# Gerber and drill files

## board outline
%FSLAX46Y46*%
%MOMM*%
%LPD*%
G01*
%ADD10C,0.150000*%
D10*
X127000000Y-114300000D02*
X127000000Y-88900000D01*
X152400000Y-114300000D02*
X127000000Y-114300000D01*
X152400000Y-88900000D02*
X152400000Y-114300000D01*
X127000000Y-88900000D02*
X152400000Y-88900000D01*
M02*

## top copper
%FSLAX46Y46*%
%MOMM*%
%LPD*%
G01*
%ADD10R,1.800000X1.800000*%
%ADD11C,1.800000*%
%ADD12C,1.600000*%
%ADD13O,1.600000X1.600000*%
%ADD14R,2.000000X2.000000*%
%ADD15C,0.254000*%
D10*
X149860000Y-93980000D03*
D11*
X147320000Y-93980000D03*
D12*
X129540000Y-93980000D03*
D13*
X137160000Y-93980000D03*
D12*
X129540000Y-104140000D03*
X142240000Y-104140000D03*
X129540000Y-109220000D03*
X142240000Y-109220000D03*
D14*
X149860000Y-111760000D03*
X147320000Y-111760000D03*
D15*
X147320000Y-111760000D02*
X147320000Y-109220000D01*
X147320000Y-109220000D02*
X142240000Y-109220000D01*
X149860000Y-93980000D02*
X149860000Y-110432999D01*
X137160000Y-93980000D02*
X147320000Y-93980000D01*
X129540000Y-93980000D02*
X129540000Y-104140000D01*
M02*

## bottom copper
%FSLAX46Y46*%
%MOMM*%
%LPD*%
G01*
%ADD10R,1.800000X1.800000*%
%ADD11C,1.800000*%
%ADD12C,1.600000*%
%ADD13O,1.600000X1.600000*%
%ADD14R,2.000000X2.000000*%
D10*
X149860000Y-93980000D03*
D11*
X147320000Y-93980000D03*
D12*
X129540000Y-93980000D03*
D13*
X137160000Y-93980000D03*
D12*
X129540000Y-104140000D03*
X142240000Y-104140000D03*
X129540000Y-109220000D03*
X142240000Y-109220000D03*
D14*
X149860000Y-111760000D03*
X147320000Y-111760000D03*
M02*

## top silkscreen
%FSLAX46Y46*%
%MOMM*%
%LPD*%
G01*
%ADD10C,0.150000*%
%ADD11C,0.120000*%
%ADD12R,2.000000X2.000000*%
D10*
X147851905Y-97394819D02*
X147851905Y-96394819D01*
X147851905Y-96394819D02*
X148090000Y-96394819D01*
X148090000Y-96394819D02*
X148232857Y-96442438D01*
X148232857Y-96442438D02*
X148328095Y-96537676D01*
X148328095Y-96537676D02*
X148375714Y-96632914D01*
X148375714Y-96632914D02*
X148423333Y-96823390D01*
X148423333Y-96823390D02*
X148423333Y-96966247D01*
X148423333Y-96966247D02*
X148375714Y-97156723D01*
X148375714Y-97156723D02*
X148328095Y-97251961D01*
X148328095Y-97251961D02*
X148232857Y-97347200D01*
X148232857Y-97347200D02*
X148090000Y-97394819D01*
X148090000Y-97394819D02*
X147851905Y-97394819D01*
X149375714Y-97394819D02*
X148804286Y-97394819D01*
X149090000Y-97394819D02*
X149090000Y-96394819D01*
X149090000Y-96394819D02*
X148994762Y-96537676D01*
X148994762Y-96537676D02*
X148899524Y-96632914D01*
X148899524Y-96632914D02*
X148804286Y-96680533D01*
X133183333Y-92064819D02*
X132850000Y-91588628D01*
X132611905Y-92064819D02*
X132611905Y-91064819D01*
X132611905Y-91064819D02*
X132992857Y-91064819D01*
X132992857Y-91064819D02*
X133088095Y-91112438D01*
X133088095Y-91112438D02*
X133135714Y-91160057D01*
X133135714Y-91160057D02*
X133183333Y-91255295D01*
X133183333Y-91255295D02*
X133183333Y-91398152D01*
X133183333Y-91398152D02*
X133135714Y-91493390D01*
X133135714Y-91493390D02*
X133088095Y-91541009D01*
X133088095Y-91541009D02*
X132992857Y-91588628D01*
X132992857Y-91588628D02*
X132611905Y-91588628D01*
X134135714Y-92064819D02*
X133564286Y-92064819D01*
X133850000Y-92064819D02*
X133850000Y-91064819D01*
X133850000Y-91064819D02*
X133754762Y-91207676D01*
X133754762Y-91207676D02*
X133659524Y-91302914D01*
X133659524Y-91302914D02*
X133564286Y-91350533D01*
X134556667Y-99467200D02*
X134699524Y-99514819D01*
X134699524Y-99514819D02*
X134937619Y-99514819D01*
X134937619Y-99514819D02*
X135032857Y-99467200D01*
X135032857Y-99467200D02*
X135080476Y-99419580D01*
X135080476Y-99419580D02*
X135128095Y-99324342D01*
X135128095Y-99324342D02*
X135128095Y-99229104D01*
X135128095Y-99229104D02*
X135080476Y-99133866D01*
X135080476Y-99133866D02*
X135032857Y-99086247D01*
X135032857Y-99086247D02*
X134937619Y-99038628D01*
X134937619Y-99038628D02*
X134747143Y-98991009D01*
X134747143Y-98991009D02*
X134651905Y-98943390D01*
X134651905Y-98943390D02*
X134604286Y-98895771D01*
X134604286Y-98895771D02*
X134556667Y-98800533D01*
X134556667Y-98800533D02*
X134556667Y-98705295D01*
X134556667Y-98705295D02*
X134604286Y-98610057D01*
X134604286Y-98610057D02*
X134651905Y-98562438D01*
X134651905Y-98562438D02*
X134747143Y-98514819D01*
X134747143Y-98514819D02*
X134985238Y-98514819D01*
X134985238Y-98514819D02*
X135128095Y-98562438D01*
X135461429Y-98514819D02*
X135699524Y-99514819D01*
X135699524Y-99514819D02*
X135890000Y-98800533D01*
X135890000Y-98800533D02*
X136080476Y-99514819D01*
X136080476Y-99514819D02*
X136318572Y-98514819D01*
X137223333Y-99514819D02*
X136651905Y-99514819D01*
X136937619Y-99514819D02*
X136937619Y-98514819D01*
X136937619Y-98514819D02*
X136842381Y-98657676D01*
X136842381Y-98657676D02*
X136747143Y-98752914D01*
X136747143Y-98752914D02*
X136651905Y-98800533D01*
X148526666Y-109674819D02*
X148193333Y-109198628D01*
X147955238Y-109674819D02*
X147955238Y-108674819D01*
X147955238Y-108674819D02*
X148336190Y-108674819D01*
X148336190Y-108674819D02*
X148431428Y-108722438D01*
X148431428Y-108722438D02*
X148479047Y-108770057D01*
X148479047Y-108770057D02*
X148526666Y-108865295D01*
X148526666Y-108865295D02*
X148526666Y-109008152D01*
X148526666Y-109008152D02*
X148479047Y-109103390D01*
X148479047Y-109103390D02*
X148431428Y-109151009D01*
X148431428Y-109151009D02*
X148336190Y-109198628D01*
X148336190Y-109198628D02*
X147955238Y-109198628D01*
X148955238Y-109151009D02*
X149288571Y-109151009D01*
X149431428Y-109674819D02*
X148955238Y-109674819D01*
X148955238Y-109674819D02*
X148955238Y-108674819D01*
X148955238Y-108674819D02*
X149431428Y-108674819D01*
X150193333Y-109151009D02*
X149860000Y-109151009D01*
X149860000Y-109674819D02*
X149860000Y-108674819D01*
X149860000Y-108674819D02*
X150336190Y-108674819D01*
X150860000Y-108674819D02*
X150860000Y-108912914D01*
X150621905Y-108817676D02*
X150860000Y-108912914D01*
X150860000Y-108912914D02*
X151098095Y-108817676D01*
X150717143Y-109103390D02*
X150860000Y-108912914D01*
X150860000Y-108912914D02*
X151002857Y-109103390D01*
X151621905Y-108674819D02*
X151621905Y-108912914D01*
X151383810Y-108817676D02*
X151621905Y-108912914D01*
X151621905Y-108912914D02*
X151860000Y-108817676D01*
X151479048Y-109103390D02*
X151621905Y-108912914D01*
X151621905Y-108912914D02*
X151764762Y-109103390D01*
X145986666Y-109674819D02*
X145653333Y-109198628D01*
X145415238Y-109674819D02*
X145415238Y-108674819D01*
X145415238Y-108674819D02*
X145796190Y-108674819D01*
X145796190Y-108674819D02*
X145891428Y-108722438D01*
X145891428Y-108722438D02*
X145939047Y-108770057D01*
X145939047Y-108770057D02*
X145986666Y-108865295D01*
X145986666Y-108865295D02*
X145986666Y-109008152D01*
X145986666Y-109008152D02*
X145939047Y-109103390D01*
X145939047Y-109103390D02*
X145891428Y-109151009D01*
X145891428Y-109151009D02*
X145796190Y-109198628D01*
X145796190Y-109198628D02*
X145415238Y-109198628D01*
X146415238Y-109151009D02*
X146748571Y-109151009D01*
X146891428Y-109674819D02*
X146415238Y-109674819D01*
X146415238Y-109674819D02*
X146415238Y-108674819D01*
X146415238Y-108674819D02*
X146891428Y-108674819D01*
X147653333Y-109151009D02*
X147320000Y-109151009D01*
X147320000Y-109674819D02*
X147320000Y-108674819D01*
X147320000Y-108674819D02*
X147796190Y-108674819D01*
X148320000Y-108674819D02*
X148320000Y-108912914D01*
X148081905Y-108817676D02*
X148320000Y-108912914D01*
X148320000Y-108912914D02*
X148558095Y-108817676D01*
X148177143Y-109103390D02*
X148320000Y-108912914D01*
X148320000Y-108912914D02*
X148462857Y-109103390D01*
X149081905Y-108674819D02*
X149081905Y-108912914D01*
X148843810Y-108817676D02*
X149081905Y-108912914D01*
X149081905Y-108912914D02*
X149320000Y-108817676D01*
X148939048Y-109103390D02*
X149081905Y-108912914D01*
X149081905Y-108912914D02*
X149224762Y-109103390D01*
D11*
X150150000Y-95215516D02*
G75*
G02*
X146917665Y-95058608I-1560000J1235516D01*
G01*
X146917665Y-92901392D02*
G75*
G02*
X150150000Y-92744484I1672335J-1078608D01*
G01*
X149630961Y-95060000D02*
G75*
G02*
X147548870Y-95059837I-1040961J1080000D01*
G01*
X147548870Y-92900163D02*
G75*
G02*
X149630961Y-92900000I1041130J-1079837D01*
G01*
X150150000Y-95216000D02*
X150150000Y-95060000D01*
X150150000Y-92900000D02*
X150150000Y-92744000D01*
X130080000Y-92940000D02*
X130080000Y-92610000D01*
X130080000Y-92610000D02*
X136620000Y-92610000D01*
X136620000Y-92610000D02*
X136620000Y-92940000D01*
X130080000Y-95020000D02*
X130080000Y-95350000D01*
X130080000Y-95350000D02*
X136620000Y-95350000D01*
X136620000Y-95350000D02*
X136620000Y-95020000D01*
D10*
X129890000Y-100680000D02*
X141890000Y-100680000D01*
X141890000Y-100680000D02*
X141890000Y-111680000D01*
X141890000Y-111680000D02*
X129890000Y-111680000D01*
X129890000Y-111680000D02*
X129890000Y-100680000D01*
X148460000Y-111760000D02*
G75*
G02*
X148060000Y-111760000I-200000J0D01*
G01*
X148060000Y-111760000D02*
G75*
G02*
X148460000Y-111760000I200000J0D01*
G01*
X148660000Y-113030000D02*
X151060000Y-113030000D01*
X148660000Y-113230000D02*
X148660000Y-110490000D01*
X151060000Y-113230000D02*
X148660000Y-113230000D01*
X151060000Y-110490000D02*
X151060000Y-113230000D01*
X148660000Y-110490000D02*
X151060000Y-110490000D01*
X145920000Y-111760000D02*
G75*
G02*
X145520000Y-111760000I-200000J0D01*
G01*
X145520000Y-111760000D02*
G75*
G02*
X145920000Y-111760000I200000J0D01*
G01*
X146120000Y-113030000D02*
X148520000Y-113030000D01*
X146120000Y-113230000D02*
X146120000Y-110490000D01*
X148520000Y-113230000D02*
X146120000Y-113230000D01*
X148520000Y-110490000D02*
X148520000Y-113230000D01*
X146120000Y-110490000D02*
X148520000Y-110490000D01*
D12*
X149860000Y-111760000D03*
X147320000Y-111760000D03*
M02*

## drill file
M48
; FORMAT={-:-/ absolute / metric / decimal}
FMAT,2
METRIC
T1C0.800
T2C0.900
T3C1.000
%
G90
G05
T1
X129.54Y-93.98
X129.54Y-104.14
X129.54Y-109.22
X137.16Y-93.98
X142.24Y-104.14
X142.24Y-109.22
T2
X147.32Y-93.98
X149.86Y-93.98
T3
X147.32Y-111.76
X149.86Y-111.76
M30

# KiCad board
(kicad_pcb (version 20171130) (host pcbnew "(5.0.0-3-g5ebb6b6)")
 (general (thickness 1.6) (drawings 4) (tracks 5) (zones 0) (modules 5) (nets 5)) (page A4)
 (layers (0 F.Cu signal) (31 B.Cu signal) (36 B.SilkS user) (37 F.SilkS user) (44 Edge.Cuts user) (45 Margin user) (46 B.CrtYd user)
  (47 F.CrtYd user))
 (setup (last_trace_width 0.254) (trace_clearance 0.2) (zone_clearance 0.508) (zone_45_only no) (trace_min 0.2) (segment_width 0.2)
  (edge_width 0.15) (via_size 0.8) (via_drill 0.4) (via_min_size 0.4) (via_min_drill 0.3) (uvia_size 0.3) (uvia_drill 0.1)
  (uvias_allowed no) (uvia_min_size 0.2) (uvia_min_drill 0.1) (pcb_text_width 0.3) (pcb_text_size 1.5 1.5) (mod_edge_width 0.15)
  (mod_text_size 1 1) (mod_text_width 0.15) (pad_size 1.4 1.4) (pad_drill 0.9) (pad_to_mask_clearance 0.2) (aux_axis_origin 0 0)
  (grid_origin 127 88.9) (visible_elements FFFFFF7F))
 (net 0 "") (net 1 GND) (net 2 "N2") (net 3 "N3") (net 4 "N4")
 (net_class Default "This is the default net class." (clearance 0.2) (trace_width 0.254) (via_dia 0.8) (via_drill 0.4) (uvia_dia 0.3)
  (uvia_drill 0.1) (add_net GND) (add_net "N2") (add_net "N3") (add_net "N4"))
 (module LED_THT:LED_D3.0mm (layer F.Cu) (at 149.86 93.98 180)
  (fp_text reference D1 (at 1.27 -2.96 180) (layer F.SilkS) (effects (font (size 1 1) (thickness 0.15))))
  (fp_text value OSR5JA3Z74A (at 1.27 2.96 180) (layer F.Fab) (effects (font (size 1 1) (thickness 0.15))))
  (fp_arc (start 1.27 0) (end -0.29 -1.235516) (angle 108.8) (layer F.SilkS) (width 0.12))
  (fp_arc (start 1.27 0) (end -0.29 1.235516) (angle -108.8) (layer F.SilkS) (width 0.12))
  (fp_arc (start 1.27 0) (end 0.229039 -1.08) (angle 87.9) (layer F.SilkS) (width 0.12))
  (fp_arc (start 1.27 0) (end 0.229039 1.08) (angle -87.9) (layer F.SilkS) (width 0.12))
  (fp_line (start -0.29 -1.236) (end -0.29 -1.08) (layer F.SilkS) (width 0.12))
  (fp_line (start -0.29 1.08) (end -0.29 1.236) (layer F.SilkS) (width 0.12))
  (pad 1 thru_hole rect (at 0 0 180) (size 1.8 1.8) (drill 0.9) (layers *.Cu *.Mask) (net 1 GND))
  (pad 2 thru_hole circle (at 2.54 0 180) (size 1.8 1.8) (drill 0.9) (layers *.Cu *.Mask) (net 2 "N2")))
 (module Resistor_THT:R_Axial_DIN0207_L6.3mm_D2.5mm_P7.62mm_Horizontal (layer F.Cu) (at 129.54 93.98)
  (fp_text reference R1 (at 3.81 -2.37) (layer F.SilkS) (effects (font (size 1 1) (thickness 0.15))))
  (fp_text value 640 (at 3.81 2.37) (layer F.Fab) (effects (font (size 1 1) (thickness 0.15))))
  (fp_line (start 0.54 -1.04) (end 0.54 -1.37) (layer F.SilkS) (width 0.12))
  (fp_line (start 0.54 -1.37) (end 7.08 -1.37) (layer F.SilkS) (width 0.12))
  (fp_line (start 7.08 -1.37) (end 7.08 -1.04) (layer F.SilkS) (width 0.12))
  (fp_line (start 0.54 1.04) (end 0.54 1.37) (layer F.SilkS) (width 0.12))
  (fp_line (start 0.54 1.37) (end 7.08 1.37) (layer F.SilkS) (width 0.12))
  (fp_line (start 7.08 1.37) (end 7.08 1.04) (layer F.SilkS) (width 0.12))
  (pad 1 thru_hole circle (at 0 0) (size 1.6 1.6) (drill 0.8) (layers *.Cu *.Mask) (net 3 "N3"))
  (pad 2 thru_hole oval (at 7.62 0) (size 1.6 1.6) (drill 0.8) (layers *.Cu *.Mask) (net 2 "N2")))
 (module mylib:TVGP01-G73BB (layer F.Cu) (at 135.89 106.68)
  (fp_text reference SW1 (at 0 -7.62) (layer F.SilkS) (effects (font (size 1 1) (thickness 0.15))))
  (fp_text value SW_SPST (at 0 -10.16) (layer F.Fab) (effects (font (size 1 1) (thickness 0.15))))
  (fp_line (start -6 -6) (end 6 -6) (layer F.SilkS) (width 0.15))
  (fp_line (start 6 -6) (end 6 5) (layer F.SilkS) (width 0.15))
  (fp_line (start 6 5) (end -6 5) (layer F.SilkS) (width 0.15))
  (fp_line (start -6 5) (end -6 -6) (layer F.SilkS) (width 0.15))
  (pad 1 thru_hole circle (at -6.35 -2.54) (size 1.6 1.6) (drill 0.8) (layers *.Cu *.Mask) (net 3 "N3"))
  (pad 2 thru_hole circle (at 6.35 -2.54) (size 1.6 1.6) (drill 0.8) (layers *.Cu *.Mask) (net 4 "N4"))
  (pad 3 thru_hole circle (at -6.35 2.54) (size 1.6 1.6) (drill 0.8) (layers *.Cu *.Mask))
  (pad 4 thru_hole circle (at 6.35 2.54) (size 1.6 1.6) (drill 0.8) (layers *.Cu *.Mask)))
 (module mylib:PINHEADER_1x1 (layer F.Cu) (at 149.86 111.76)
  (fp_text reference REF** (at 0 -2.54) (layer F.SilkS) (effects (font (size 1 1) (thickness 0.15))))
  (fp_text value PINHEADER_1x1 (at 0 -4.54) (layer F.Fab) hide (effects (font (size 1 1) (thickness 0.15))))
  (fp_circle (center -1.6 0) (end -1.6 0.2) (layer F.SilkS) (width 0.15))
  (fp_line (start -1.2 1.27) (end 1.2 1.27) (layer F.SilkS) (width 0.15))
  (fp_line (start -1.2 1.47) (end -1.2 -1.27) (layer F.SilkS) (width 0.15))
  (fp_line (start 1.2 1.47) (end -1.2 1.47) (layer F.SilkS) (width 0.15))
  (fp_line (start 1.2 -1.27) (end 1.2 1.47) (layer F.SilkS) (width 0.15))
  (fp_line (start -1.2 -1.27) (end 1.2 -1.27) (layer F.SilkS) (width 0.15))
  (pad 1 thru_hole rect (at 0 0) (size 2 2) (drill 1) (layers *.Cu *.Mask F.SilkS)))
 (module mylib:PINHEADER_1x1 (layer F.Cu) (at 147.32 111.76)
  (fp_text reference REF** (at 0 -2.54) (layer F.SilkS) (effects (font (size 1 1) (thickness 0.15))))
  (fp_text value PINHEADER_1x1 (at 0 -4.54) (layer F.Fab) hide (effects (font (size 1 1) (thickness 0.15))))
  (fp_circle (center -1.6 0) (end -1.6 0.2) (layer F.SilkS) (width 0.15))
  (fp_line (start -1.2 1.27) (end 1.2 1.27) (layer F.SilkS) (width 0.15))
  (fp_line (start -1.2 1.47) (end -1.2 -1.27) (layer F.SilkS) (width 0.15))
  (fp_line (start 1.2 1.47) (end -1.2 1.47) (layer F.SilkS) (width 0.15))
  (fp_line (start 1.2 -1.27) (end 1.2 1.47) (layer F.SilkS) (width 0.15))
  (fp_line (start -1.2 -1.27) (end 1.2 -1.27) (layer F.SilkS) (width 0.15))
  (pad 1 thru_hole rect (at 0 0) (size 2 2) (drill 1) (layers *.Cu *.Mask F.SilkS)))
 (gr_line (start 127 114.3) (end 127 88.9) (layer Edge.Cuts) (width 0.15))
 (gr_line (start 152.4 114.3) (end 127 114.3) (layer Edge.Cuts) (width 0.15))
 (gr_line (start 152.4 88.9) (end 152.4 114.3) (layer Edge.Cuts) (width 0.15))
 (gr_line (start 127 88.9) (end 152.4 88.9) (layer Edge.Cuts) (width 0.15))
 (segment (start 147.32 111.76) (end 147.32 109.22) (width 0.254) (layer F.Cu) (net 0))
 (segment (start 147.32 109.22) (end 142.24 109.22) (width 0.254) (layer F.Cu) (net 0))
 (segment (start 149.86 93.98) (end 149.86 110.432999) (width 0.254) (layer F.Cu) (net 1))
 (segment (start 137.16 93.98) (end 147.32 93.98) (width 0.254) (layer F.Cu) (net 2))
 (segment (start 129.54 93.98) (end 129.54 104.14) (width 0.254) (layer F.Cu) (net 3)))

